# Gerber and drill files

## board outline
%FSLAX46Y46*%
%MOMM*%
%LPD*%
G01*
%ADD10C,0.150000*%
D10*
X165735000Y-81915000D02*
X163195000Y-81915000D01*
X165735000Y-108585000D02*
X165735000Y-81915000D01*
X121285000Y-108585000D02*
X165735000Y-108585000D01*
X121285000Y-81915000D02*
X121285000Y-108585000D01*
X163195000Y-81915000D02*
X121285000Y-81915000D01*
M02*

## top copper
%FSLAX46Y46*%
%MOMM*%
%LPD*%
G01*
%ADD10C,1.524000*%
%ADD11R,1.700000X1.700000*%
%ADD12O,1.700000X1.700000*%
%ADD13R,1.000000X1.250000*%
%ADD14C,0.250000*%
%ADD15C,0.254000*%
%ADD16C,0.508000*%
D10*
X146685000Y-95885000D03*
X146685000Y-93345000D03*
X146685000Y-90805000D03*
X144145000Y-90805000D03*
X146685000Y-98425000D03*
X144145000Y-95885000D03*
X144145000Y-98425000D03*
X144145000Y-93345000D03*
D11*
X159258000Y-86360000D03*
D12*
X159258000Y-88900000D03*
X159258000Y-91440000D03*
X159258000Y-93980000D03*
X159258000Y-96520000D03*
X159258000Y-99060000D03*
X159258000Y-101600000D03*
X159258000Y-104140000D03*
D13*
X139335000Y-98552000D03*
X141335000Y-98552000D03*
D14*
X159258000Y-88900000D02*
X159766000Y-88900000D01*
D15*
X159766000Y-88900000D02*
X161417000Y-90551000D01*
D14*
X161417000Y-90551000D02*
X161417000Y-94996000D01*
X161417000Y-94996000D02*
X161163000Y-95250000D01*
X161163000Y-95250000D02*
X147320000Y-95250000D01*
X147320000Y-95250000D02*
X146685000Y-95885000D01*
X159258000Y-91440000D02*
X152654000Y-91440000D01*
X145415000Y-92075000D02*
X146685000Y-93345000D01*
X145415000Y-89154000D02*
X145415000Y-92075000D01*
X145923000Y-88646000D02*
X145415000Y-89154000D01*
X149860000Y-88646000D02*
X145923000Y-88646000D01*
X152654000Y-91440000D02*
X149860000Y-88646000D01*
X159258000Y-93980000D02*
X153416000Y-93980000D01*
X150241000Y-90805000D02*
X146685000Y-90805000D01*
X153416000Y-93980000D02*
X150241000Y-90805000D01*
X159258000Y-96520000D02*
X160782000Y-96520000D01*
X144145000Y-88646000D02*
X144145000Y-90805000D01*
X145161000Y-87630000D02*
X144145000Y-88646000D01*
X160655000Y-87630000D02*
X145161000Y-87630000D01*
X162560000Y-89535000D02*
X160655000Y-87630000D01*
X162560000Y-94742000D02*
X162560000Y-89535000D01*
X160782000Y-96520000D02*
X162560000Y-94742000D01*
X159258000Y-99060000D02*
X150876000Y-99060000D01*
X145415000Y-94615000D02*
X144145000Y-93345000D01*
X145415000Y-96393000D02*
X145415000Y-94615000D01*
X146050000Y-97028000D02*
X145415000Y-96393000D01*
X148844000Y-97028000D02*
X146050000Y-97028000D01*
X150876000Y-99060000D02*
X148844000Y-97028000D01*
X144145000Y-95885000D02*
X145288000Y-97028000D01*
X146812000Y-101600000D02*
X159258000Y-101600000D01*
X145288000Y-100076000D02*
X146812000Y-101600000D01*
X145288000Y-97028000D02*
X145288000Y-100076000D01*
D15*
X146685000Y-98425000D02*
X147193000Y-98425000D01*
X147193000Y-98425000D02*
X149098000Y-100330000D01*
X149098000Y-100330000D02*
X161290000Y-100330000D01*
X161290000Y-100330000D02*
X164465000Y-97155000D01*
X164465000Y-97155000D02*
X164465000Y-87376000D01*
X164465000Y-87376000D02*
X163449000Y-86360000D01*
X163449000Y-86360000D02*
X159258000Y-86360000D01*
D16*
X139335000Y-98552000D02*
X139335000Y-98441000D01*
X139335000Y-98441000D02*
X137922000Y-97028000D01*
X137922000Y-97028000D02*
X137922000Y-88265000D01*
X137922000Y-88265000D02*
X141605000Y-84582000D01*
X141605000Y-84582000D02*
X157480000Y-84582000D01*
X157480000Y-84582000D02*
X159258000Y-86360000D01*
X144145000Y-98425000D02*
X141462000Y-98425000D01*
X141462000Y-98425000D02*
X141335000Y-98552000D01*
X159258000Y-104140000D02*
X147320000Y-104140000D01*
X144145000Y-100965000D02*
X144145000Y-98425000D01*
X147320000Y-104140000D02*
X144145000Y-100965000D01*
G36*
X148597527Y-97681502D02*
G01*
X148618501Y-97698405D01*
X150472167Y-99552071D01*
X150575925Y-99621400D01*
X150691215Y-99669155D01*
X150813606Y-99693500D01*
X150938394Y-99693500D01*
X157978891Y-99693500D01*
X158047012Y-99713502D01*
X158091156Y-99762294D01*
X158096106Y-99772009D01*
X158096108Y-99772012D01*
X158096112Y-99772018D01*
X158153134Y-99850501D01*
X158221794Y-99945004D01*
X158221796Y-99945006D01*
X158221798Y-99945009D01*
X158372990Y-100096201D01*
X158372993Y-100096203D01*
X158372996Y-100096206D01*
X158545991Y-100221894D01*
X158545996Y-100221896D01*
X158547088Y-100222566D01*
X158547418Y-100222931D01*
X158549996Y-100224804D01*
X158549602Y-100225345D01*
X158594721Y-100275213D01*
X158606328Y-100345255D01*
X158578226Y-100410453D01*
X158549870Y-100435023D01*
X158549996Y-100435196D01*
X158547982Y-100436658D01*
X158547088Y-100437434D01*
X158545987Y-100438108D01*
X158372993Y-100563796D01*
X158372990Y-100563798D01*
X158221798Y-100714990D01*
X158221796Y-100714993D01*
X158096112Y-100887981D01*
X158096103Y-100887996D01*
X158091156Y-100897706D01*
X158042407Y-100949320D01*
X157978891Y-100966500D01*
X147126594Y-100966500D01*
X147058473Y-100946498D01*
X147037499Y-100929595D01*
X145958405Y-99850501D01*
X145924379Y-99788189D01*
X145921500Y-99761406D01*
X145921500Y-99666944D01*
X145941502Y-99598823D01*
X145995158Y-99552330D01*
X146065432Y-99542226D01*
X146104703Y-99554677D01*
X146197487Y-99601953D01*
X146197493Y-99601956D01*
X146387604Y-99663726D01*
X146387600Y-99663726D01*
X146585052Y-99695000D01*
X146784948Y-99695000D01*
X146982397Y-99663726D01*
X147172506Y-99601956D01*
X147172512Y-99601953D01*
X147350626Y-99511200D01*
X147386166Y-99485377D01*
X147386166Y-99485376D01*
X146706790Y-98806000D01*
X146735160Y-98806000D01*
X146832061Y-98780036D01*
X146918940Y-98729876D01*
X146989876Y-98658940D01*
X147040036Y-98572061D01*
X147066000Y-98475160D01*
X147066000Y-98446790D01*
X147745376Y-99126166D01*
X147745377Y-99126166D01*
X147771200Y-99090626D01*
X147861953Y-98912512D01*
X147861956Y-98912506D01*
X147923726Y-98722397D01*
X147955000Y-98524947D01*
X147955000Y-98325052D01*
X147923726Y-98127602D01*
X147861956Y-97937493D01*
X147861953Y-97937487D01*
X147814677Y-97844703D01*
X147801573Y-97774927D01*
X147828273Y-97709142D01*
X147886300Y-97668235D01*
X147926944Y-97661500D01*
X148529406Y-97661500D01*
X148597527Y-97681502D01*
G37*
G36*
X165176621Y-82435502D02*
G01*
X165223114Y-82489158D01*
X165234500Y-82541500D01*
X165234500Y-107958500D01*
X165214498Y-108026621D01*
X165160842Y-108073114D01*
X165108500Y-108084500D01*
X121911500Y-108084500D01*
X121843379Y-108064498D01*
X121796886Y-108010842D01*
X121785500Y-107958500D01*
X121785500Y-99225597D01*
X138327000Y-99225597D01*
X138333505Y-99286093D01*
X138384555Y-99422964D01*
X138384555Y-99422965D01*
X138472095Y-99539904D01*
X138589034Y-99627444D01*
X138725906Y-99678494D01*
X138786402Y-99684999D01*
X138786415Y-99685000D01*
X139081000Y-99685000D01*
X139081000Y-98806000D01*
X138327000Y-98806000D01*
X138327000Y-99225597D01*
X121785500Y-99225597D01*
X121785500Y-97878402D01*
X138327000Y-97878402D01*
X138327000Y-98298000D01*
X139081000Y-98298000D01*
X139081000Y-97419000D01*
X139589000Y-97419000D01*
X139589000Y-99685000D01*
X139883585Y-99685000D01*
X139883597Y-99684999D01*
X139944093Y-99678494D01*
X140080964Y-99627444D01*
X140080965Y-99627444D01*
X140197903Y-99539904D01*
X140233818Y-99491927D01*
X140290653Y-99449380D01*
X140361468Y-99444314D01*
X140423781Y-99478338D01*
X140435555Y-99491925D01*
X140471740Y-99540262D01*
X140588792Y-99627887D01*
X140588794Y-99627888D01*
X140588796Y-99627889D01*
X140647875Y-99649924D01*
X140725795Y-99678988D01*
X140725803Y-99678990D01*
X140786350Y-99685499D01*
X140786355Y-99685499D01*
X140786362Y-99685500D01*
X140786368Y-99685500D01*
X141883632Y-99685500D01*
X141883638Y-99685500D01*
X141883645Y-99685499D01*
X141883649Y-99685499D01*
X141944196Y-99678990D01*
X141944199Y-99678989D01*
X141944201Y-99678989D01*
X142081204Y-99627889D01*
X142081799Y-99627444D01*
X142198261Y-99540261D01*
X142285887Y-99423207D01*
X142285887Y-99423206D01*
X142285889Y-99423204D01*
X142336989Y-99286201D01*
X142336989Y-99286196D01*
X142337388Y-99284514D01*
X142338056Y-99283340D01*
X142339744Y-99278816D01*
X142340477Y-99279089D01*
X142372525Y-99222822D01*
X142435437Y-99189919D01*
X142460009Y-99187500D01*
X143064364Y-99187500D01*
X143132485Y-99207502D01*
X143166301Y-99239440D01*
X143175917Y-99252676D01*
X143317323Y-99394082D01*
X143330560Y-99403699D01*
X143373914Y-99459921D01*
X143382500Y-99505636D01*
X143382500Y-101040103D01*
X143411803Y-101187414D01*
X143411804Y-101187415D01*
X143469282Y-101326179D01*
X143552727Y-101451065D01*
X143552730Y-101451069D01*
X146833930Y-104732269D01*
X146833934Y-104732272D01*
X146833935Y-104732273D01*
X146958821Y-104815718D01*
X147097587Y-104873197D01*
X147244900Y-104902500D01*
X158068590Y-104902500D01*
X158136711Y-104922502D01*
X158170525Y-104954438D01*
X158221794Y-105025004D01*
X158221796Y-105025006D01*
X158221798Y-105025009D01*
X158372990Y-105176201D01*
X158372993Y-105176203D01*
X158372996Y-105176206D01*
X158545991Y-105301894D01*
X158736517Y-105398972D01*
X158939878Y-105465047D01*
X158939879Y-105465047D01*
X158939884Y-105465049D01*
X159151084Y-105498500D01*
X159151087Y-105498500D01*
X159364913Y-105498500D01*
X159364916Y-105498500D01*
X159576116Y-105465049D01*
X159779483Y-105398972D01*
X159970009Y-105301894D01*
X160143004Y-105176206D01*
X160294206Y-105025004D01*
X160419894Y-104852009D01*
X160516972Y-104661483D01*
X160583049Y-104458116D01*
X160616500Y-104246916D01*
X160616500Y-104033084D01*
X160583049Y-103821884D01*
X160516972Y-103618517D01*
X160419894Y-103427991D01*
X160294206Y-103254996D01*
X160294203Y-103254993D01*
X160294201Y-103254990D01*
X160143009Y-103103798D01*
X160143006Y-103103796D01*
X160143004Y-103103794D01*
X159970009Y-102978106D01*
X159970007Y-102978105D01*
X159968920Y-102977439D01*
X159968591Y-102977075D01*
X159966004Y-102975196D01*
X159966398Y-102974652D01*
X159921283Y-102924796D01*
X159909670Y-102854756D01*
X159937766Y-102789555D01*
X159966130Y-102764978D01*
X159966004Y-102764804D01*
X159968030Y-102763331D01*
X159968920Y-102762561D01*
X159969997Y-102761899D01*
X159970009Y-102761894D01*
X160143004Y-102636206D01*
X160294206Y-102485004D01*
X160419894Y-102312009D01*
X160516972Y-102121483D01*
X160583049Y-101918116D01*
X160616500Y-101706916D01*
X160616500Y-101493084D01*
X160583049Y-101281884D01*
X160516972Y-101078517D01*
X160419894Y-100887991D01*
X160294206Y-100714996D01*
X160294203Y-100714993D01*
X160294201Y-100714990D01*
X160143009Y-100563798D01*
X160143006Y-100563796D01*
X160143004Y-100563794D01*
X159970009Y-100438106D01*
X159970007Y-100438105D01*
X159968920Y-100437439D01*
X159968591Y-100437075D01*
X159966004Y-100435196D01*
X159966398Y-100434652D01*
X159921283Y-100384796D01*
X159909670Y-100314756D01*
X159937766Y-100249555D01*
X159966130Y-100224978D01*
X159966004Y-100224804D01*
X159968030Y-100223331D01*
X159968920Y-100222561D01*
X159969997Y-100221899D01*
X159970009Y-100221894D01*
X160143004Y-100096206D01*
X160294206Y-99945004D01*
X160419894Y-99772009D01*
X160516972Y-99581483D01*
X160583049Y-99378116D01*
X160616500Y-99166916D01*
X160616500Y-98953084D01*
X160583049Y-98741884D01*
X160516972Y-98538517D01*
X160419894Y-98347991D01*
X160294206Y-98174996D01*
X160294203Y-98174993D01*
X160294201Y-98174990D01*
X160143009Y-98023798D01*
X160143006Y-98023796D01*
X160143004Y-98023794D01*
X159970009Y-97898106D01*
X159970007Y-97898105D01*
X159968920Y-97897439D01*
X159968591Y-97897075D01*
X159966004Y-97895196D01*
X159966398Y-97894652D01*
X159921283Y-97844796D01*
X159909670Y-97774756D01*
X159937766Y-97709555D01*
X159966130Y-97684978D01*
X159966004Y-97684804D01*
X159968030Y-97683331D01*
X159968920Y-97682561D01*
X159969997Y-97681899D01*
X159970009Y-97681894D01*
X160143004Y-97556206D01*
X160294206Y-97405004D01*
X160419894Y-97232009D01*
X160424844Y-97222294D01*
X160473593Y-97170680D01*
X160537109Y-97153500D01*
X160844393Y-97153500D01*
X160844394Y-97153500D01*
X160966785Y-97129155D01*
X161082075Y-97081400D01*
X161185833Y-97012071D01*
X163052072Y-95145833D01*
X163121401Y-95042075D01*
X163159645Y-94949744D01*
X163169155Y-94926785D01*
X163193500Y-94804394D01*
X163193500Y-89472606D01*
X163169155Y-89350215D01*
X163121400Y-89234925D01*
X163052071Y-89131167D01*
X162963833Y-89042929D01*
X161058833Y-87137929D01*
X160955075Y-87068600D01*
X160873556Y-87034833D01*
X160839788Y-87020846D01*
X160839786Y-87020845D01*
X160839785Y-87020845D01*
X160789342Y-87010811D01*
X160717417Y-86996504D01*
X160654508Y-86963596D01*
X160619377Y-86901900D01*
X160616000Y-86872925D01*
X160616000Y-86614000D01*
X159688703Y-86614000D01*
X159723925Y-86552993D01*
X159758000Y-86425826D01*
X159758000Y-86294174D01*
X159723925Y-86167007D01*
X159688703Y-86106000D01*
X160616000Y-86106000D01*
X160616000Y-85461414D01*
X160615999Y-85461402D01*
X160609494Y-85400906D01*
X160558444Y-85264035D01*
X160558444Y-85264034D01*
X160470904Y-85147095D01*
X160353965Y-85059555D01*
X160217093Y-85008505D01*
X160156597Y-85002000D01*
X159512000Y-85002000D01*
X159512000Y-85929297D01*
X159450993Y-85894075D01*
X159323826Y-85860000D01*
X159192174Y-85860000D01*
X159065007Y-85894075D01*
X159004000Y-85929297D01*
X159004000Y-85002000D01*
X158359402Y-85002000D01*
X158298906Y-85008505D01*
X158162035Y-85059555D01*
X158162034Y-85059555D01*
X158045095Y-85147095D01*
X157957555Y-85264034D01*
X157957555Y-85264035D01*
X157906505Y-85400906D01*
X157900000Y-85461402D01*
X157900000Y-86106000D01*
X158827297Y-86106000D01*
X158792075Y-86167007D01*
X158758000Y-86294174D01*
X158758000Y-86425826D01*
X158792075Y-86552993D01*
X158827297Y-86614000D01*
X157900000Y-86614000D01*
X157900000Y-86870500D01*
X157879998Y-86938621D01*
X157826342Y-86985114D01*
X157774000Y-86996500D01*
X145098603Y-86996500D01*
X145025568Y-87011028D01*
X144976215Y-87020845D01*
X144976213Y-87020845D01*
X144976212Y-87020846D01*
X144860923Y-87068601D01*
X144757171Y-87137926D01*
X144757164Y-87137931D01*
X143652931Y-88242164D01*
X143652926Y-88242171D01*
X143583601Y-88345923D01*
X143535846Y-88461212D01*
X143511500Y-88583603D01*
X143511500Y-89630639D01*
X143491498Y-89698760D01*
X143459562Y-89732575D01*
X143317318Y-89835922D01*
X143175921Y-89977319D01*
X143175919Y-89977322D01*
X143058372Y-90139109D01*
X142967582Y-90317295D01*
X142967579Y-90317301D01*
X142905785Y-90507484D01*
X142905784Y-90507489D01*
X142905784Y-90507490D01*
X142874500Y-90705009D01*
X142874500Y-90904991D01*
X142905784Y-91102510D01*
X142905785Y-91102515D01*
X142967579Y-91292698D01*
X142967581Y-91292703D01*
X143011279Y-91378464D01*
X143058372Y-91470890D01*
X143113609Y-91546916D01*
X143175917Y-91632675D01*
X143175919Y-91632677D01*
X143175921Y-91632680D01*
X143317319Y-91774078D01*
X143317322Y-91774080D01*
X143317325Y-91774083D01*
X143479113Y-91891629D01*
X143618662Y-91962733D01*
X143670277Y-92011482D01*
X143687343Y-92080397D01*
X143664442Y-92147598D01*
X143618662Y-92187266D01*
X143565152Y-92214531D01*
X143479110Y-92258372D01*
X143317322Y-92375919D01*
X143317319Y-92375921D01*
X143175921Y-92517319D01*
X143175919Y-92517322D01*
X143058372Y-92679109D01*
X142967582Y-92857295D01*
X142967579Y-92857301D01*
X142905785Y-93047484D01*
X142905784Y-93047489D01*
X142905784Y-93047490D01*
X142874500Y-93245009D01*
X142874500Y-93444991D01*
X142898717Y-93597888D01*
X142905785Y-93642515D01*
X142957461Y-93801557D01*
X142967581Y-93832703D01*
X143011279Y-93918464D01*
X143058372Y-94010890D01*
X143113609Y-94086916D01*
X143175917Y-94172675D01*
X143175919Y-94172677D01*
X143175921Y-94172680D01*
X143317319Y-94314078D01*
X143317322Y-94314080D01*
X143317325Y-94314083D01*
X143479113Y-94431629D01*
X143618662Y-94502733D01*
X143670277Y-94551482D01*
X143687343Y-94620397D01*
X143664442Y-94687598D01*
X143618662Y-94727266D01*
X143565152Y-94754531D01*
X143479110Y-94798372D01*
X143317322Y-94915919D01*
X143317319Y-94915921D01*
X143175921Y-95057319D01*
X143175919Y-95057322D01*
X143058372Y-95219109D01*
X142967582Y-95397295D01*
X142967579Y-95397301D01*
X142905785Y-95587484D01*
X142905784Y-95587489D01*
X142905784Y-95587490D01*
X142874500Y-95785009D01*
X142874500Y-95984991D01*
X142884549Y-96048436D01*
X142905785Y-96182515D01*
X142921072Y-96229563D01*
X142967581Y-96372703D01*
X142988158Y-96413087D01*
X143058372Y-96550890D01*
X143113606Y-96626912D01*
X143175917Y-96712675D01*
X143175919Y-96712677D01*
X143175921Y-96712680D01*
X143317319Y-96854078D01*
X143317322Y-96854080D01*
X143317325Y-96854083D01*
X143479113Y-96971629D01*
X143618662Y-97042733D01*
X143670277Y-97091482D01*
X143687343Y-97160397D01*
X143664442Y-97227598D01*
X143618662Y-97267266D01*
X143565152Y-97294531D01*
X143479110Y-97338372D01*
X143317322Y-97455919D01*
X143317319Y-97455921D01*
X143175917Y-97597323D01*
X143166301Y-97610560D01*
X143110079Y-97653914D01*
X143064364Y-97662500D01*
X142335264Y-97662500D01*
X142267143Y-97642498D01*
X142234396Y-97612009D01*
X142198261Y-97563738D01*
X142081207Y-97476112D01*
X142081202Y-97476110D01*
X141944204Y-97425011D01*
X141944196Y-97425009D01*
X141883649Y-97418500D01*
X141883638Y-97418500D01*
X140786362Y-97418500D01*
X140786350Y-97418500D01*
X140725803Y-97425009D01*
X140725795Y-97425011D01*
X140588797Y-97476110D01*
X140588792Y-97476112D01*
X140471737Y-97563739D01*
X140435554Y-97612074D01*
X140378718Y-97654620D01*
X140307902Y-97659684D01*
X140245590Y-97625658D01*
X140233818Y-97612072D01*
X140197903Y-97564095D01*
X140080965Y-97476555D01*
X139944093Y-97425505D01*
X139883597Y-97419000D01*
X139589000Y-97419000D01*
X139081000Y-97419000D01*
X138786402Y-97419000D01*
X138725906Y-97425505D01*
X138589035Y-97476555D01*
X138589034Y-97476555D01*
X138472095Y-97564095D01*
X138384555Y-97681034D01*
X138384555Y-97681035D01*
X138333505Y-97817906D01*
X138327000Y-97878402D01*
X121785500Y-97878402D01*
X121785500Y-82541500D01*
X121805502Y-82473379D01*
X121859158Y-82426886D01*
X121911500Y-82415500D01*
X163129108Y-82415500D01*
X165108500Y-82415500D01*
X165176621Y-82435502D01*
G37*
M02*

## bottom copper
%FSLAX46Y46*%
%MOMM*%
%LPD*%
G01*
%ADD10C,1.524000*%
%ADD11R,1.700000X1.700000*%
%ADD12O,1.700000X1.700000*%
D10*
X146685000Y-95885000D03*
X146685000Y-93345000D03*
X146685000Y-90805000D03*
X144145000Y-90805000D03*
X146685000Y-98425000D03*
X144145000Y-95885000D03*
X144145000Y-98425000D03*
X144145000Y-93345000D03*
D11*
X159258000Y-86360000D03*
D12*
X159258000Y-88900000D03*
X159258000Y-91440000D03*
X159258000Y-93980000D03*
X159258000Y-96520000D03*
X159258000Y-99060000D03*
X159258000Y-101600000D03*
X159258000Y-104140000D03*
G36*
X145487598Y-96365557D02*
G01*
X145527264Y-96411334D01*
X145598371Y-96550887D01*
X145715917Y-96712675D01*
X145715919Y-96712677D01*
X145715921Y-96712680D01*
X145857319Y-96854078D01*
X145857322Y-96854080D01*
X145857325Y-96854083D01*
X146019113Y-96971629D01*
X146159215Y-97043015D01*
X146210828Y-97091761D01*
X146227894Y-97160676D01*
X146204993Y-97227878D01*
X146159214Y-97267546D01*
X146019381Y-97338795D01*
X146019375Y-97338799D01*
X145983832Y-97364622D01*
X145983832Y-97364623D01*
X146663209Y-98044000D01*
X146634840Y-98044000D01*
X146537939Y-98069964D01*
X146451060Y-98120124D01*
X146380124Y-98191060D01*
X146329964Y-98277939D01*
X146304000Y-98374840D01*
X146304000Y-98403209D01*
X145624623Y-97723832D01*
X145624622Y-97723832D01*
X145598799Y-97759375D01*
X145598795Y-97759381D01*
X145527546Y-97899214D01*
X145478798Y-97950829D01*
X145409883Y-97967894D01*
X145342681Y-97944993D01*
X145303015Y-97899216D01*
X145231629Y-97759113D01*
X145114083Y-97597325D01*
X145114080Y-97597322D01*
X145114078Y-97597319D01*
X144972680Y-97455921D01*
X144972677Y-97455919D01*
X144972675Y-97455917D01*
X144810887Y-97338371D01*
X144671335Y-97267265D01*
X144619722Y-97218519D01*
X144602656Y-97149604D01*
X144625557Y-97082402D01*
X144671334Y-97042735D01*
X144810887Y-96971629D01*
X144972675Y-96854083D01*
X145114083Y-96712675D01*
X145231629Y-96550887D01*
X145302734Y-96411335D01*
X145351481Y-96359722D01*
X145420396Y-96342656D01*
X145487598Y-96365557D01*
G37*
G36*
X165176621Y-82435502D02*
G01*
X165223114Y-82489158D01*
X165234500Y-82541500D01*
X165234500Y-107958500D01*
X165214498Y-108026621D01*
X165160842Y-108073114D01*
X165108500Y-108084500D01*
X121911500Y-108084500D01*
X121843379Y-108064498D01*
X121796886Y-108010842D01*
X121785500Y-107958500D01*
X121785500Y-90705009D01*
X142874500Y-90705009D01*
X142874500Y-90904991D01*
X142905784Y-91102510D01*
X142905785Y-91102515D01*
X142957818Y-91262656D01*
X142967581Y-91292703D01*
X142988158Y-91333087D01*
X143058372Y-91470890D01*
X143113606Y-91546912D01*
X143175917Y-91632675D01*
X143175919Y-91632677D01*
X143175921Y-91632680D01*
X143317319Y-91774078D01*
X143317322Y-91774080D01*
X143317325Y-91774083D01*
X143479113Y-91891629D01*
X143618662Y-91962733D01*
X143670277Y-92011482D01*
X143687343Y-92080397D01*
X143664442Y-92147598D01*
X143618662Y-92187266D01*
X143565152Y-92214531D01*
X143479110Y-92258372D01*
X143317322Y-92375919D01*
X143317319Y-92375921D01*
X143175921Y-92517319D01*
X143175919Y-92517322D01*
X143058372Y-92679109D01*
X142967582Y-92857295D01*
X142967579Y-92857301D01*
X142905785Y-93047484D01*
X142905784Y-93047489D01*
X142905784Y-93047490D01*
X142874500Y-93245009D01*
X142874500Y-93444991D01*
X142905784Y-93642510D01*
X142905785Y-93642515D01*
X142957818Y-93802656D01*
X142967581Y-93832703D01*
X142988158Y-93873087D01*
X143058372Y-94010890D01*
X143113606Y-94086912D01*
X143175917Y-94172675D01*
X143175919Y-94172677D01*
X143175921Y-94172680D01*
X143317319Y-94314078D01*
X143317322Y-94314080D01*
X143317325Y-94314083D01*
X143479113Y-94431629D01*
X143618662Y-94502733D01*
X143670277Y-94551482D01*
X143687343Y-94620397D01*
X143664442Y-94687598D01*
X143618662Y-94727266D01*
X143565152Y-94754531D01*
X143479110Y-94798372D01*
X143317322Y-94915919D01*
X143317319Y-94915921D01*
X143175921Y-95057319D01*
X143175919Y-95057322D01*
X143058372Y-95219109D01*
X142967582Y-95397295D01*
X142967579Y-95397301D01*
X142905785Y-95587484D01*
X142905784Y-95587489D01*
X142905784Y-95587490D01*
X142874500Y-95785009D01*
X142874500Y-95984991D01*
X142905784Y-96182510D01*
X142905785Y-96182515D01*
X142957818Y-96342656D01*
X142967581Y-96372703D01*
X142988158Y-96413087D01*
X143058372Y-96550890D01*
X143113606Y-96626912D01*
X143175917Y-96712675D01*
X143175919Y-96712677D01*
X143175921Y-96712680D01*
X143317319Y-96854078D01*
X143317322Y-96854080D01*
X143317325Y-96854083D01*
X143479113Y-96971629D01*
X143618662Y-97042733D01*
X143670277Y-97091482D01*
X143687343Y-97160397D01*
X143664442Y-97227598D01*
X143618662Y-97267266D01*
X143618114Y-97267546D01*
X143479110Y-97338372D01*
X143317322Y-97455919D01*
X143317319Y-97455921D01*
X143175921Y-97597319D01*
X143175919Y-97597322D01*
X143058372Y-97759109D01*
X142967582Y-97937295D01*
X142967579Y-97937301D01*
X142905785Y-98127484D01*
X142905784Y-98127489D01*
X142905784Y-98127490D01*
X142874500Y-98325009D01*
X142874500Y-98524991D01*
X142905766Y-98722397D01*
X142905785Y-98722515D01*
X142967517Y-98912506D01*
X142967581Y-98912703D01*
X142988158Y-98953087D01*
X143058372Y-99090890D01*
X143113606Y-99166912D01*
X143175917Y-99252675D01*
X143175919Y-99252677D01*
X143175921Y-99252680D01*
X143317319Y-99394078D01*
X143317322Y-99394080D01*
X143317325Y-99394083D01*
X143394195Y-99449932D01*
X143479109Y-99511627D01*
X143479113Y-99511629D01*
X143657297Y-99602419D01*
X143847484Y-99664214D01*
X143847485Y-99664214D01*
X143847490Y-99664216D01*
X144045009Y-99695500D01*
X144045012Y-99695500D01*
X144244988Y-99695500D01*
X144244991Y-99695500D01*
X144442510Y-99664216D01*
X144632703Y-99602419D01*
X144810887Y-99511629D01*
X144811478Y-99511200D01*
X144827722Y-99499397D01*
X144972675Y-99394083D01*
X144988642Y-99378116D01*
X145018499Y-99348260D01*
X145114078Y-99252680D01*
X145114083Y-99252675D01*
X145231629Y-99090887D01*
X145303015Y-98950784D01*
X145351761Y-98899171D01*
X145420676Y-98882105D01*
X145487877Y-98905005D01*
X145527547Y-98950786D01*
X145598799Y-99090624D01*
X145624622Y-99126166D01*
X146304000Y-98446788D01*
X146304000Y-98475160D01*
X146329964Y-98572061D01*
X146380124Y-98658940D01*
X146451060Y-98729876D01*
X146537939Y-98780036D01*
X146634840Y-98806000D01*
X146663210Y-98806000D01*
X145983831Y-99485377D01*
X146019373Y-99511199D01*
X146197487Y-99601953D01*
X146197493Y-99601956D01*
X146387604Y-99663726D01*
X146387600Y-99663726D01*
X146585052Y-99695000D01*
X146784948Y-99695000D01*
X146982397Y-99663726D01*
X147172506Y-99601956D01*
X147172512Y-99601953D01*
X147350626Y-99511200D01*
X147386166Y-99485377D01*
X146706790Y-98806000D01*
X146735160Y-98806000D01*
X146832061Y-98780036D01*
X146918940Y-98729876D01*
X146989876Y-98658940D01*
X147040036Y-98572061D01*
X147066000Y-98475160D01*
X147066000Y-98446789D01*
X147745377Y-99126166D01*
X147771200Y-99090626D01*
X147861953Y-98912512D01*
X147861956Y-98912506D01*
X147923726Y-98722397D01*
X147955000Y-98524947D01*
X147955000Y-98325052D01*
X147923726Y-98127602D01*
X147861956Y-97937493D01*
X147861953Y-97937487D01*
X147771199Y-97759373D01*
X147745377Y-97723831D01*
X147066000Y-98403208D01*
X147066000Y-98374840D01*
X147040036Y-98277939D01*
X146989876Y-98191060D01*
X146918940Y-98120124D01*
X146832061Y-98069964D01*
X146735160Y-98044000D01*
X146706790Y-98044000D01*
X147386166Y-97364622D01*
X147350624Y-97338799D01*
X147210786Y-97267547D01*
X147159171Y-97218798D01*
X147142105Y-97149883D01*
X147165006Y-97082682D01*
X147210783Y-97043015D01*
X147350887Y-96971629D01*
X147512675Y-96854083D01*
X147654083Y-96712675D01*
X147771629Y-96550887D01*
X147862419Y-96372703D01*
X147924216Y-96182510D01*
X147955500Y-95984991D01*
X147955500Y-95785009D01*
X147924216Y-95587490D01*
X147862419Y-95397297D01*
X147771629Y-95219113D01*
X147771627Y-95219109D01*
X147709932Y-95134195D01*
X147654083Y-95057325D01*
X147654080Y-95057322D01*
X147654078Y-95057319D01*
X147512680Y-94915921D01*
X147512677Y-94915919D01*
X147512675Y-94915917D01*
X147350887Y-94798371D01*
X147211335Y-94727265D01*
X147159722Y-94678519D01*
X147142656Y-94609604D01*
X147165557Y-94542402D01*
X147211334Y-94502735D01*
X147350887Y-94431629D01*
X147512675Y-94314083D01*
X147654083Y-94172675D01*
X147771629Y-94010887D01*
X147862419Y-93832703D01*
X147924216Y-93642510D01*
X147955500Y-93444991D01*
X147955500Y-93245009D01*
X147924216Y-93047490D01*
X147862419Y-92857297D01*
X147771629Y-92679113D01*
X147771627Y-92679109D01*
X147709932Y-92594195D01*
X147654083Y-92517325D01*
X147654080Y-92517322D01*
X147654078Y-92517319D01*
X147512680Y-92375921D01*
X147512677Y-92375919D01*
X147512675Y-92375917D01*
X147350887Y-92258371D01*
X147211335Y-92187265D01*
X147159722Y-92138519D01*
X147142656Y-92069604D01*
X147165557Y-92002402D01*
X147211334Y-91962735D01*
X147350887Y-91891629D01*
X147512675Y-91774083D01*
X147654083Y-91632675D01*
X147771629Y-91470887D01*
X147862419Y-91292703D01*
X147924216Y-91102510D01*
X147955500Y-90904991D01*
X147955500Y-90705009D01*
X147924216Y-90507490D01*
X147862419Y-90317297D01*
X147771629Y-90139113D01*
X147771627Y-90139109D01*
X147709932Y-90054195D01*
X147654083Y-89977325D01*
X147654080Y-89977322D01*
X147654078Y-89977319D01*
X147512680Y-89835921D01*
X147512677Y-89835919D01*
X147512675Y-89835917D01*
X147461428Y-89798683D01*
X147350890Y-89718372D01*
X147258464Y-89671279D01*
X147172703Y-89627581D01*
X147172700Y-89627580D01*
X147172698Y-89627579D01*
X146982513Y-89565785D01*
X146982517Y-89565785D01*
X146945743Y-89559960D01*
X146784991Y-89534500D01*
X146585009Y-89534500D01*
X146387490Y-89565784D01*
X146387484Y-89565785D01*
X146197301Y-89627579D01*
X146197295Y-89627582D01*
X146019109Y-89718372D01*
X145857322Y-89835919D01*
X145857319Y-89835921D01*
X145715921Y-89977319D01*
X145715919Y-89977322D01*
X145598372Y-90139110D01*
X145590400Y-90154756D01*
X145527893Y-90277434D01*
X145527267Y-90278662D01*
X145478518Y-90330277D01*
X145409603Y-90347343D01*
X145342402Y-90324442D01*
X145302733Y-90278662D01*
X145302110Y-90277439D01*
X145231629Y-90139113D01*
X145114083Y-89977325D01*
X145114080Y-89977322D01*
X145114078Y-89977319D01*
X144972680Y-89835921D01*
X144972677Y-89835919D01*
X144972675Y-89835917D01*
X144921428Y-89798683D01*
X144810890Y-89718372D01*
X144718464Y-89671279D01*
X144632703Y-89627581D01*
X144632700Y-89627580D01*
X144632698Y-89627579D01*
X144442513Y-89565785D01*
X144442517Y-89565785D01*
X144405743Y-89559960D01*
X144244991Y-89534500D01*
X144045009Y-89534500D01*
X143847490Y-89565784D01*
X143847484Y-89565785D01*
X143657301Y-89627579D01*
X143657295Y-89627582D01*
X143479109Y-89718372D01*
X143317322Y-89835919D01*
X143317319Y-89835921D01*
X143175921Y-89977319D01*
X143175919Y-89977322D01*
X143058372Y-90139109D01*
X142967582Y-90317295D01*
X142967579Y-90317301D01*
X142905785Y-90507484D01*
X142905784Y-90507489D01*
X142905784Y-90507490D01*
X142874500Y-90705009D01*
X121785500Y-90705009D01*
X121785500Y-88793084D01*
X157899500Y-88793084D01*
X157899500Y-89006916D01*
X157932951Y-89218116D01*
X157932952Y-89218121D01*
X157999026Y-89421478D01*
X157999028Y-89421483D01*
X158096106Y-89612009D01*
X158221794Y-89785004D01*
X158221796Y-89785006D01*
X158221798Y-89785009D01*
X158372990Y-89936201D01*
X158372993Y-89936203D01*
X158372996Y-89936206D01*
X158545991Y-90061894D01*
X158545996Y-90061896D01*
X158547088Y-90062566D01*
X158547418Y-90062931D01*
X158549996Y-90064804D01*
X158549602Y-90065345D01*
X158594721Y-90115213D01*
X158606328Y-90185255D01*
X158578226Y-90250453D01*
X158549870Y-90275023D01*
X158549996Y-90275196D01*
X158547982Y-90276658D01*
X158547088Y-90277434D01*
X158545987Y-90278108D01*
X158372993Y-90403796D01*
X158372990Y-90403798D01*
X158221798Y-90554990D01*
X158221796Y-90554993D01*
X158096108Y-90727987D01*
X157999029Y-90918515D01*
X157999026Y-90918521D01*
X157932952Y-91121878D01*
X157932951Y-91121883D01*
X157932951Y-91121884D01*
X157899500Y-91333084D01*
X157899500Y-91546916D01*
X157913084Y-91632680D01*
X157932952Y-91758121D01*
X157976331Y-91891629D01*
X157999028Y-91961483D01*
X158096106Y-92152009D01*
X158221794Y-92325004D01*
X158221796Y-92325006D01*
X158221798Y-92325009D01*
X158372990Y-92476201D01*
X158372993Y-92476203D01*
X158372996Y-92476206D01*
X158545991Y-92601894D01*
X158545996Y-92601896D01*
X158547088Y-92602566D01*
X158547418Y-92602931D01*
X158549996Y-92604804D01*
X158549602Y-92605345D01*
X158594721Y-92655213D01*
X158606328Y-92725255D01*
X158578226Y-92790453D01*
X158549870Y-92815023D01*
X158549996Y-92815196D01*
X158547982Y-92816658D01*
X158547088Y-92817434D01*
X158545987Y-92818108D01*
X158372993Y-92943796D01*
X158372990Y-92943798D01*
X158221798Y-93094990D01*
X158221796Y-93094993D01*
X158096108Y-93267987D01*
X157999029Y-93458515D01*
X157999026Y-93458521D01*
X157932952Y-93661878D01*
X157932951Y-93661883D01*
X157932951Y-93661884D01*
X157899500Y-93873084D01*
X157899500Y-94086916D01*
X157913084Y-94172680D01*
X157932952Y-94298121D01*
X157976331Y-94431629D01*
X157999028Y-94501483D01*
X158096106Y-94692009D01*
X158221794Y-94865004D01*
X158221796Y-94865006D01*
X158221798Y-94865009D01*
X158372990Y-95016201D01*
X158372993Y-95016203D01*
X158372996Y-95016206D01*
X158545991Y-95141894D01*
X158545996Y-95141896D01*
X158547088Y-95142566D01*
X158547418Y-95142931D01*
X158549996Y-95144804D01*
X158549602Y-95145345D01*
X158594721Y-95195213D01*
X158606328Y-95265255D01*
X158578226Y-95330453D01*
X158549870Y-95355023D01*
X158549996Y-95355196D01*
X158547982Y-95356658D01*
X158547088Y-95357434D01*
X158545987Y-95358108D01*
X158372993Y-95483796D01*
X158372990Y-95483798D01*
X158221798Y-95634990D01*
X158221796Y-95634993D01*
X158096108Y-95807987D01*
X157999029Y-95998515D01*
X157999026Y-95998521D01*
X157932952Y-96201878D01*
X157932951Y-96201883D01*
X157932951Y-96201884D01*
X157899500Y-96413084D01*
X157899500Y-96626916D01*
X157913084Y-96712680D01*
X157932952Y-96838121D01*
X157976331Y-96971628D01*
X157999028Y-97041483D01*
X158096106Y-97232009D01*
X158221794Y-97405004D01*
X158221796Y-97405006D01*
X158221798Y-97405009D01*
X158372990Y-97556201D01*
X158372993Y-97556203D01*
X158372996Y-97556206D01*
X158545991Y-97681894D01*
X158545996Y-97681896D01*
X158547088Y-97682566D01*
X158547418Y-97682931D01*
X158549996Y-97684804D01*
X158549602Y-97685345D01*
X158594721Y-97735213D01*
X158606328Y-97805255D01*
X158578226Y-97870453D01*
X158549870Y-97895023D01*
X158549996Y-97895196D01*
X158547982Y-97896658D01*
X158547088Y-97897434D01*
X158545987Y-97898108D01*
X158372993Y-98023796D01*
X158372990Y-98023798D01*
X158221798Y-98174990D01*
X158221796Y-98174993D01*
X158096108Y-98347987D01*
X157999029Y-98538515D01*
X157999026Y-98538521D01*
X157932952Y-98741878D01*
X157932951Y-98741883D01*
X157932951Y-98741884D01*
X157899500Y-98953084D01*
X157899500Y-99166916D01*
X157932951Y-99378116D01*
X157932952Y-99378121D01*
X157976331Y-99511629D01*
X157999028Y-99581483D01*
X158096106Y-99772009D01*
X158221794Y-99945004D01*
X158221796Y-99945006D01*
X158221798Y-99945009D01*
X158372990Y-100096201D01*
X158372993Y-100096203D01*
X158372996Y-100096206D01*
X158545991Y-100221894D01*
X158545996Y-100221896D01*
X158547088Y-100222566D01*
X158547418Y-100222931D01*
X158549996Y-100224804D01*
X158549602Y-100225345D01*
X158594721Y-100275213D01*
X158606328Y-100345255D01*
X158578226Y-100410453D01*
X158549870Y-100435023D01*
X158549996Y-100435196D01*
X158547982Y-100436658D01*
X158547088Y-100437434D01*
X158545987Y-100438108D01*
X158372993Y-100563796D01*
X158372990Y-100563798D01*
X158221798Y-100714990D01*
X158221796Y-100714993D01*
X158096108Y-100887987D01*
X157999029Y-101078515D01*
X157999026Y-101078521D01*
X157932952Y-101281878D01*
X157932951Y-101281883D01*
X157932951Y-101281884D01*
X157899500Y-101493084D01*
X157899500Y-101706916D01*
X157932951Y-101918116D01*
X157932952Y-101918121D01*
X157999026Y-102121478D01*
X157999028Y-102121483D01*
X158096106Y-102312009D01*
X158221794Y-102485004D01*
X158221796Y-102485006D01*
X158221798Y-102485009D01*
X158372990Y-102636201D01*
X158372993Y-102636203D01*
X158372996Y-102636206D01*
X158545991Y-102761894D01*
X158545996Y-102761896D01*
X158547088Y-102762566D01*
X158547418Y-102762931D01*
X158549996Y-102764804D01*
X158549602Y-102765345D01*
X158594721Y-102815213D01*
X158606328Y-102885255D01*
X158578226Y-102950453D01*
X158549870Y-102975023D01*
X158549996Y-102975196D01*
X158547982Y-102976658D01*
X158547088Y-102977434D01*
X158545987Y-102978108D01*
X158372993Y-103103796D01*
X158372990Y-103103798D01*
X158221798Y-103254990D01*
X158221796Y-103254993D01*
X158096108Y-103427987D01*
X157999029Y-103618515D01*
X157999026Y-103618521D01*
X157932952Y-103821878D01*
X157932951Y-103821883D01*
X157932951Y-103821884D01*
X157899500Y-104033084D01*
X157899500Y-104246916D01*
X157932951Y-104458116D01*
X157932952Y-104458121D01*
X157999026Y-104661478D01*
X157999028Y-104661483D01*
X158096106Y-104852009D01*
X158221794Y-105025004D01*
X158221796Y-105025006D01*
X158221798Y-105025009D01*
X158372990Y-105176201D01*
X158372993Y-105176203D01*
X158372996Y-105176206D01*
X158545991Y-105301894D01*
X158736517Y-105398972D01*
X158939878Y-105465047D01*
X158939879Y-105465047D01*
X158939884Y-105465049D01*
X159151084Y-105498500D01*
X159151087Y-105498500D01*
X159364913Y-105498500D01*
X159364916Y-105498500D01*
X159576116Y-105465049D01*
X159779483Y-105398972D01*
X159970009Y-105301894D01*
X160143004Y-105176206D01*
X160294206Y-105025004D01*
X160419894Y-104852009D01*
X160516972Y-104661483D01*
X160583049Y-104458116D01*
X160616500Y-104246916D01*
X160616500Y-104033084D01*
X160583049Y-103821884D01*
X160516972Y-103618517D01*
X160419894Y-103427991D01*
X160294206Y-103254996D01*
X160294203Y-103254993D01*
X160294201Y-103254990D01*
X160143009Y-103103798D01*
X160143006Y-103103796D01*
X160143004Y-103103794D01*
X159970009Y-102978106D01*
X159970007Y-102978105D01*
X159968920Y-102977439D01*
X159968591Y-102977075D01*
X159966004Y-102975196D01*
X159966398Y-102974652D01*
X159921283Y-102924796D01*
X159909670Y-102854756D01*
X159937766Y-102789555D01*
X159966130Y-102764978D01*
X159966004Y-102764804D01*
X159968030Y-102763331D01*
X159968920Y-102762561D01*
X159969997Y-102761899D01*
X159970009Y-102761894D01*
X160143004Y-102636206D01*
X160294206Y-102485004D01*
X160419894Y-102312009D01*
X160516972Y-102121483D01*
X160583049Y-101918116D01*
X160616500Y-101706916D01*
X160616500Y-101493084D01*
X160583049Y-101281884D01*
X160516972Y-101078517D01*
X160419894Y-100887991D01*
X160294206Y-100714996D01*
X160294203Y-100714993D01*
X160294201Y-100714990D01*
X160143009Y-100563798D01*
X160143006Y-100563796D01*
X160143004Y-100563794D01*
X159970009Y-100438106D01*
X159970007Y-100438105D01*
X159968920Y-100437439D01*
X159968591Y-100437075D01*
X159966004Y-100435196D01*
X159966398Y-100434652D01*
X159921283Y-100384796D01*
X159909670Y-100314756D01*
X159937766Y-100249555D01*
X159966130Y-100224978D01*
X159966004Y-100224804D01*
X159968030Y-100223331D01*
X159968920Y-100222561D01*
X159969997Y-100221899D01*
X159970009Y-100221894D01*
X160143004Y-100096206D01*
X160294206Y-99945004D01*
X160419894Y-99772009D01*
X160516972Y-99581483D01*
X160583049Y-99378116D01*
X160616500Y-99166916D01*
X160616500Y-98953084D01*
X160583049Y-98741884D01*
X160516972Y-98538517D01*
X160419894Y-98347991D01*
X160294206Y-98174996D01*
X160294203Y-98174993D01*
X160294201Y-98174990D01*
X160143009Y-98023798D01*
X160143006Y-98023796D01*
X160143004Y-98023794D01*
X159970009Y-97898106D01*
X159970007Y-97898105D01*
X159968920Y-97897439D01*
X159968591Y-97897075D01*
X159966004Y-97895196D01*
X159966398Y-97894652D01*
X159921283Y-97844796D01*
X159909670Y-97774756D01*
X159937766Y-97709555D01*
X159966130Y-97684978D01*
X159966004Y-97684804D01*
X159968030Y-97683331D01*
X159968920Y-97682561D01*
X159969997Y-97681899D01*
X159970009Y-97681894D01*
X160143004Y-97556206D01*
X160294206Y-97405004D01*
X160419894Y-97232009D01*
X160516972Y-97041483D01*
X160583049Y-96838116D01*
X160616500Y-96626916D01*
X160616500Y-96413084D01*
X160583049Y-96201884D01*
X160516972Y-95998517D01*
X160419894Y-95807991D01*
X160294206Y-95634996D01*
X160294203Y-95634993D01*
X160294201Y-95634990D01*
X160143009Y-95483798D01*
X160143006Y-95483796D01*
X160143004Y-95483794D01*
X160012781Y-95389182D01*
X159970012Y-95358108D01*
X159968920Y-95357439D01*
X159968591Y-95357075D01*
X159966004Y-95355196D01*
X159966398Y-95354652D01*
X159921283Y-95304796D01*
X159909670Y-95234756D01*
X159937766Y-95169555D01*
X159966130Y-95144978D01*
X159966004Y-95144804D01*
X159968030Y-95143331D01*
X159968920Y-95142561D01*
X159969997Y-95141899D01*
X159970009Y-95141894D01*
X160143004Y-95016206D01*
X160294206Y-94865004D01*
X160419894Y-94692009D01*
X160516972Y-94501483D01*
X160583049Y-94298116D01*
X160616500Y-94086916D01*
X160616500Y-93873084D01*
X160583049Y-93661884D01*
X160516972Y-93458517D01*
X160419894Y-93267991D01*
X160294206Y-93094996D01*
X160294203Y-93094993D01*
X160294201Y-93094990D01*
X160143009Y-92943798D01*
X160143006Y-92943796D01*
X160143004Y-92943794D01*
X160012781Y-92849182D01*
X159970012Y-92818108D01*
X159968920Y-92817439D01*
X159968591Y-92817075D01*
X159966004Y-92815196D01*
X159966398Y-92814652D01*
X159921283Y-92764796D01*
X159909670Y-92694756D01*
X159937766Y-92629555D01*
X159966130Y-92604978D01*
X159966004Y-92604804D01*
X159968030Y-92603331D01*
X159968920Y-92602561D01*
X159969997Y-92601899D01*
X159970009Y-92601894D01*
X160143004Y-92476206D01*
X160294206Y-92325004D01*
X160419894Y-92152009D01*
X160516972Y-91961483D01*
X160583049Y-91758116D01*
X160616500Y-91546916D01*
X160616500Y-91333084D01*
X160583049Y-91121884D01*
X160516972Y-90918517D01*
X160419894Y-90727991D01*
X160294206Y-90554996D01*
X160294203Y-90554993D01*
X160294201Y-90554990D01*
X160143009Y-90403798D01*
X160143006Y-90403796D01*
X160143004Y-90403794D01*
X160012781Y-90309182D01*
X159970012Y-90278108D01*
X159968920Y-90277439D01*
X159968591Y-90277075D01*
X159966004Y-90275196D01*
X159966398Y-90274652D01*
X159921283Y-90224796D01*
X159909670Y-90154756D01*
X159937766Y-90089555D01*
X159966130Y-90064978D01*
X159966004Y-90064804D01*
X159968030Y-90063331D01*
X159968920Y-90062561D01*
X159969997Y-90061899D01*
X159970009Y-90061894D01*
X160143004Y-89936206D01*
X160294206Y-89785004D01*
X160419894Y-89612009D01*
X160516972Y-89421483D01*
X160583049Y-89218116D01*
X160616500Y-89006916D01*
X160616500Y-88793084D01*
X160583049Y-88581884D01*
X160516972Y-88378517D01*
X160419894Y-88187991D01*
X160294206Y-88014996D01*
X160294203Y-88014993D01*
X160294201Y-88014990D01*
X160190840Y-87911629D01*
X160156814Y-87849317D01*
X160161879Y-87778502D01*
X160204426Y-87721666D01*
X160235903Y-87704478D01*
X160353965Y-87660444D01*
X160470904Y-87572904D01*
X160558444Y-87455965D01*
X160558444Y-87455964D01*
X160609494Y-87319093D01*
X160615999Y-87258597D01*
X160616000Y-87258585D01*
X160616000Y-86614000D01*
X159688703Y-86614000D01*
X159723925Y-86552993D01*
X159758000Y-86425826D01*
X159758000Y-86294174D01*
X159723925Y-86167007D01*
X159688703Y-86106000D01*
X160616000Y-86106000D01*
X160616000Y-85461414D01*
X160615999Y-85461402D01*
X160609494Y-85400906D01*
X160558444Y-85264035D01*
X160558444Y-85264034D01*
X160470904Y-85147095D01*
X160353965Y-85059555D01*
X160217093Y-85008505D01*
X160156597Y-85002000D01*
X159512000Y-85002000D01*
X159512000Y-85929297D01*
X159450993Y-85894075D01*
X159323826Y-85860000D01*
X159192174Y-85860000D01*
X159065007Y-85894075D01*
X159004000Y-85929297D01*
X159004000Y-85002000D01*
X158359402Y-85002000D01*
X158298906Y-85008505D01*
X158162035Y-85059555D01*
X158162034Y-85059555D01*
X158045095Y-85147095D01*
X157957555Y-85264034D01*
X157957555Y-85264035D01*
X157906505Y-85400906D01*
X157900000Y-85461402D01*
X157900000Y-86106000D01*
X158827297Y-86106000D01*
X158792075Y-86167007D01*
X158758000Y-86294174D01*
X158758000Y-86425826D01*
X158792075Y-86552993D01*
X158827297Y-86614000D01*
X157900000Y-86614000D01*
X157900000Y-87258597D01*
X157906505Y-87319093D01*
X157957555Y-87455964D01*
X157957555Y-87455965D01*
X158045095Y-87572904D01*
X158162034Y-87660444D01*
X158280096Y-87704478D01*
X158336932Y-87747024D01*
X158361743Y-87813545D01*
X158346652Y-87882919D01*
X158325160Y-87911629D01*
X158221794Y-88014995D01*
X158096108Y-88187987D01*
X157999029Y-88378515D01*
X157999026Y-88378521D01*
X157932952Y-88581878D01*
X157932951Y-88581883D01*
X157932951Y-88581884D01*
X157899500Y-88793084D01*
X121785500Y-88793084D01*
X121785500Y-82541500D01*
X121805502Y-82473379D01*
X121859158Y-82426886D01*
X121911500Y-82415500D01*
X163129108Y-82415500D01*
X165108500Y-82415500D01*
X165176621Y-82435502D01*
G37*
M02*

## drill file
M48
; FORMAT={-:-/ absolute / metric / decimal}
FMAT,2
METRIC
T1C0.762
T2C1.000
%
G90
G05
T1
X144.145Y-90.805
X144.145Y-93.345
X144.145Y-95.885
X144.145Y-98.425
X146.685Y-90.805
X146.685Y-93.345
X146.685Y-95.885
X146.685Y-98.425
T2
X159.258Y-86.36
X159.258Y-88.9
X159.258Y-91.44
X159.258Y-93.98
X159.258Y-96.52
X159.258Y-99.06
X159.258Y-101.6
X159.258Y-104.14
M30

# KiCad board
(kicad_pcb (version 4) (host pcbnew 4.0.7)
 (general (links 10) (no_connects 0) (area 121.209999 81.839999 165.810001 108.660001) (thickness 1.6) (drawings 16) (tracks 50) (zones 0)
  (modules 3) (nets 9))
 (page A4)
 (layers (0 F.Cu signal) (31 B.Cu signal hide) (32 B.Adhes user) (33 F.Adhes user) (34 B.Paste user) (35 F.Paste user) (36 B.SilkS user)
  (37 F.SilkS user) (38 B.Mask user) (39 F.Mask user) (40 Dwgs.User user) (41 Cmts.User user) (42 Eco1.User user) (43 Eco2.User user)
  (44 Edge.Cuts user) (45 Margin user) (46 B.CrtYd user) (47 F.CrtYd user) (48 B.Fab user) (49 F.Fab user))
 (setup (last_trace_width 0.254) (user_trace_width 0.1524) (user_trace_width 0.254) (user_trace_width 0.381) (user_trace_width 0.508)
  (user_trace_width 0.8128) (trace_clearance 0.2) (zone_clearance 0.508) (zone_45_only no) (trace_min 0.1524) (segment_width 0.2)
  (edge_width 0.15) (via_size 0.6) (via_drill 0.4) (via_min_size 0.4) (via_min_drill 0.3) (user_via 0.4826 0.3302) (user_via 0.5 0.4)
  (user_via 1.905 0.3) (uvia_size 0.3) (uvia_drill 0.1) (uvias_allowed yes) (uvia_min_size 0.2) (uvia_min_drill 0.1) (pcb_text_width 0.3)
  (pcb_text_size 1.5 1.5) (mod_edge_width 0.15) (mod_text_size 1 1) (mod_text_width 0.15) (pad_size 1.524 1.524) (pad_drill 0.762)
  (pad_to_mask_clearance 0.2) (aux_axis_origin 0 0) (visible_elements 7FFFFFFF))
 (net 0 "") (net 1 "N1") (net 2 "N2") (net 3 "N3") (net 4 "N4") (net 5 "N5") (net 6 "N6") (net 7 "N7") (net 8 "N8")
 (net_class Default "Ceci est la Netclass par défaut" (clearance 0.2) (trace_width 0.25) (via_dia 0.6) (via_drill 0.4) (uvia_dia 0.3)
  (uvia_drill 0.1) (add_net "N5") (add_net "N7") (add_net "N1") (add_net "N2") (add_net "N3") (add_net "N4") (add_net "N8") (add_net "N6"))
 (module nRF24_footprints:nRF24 (layer F.Cu) (at 139.065 95.885)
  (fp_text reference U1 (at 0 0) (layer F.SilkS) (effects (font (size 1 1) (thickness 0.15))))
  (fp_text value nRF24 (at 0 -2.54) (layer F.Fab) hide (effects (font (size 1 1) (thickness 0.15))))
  (pad 1 thru_hole circle (at 7.62 0) (size 1.524 1.524) (drill 0.762) (layers *.Cu *.Mask) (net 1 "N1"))
  (pad 2 thru_hole circle (at 7.62 -2.54) (size 1.524 1.524) (drill 0.762) (layers *.Cu *.Mask) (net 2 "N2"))
  (pad 3 thru_hole circle (at 7.62 -5.08) (size 1.524 1.524) (drill 0.762) (layers *.Cu *.Mask) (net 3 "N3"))
  (pad 4 thru_hole circle (at 5.08 -5.08) (size 1.524 1.524) (drill 0.762) (layers *.Cu *.Mask) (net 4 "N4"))
  (pad 0 thru_hole circle (at 7.62 2.54) (size 1.524 1.524) (drill 0.762) (layers *.Cu *.Mask) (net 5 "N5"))
  (pad 6 thru_hole circle (at 5.08 0) (size 1.524 1.524) (drill 0.762) (layers *.Cu *.Mask) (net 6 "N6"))
  (pad 7 thru_hole circle (at 5.08 2.54) (size 1.524 1.524) (drill 0.762) (layers *.Cu *.Mask) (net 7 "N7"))
  (pad 5 thru_hole circle (at 5.08 -2.54) (size 1.524 1.524) (drill 0.762) (layers *.Cu *.Mask) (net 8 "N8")))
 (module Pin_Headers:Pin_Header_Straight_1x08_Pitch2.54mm (layer F.Cu) (at 159.258 86.36)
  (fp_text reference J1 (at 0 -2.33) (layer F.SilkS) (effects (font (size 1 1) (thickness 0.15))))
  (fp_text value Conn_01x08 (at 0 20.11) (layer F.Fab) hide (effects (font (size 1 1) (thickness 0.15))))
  (pad 1 thru_hole rect (at 0 0) (size 1.7 1.7) (drill 1) (layers *.Cu *.Mask) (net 5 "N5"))
  (pad 2 thru_hole oval (at 0 2.54) (size 1.7 1.7) (drill 1) (layers *.Cu *.Mask) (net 1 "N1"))
  (pad 3 thru_hole oval (at 0 5.08) (size 1.7 1.7) (drill 1) (layers *.Cu *.Mask) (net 2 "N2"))
  (pad 4 thru_hole oval (at 0 7.62) (size 1.7 1.7) (drill 1) (layers *.Cu *.Mask) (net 3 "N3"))
  (pad 5 thru_hole oval (at 0 10.16) (size 1.7 1.7) (drill 1) (layers *.Cu *.Mask) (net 4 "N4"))
  (pad 6 thru_hole oval (at 0 12.7) (size 1.7 1.7) (drill 1) (layers *.Cu *.Mask) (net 8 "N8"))
  (pad 7 thru_hole oval (at 0 15.24) (size 1.7 1.7) (drill 1) (layers *.Cu *.Mask) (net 6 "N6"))
  (pad 8 thru_hole oval (at 0 17.78) (size 1.7 1.7) (drill 1) (layers *.Cu *.Mask) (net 7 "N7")))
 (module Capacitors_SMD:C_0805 (layer F.Cu) (at 140.335 98.552)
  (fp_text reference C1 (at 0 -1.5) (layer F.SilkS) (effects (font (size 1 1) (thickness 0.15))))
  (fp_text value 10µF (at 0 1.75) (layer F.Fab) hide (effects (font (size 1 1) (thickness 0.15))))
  (pad 1 smd rect (at -1 0) (size 1 1.25) (layers F.Cu F.Paste F.Mask) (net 5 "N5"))
  (pad 2 smd rect (at 1 0) (size 1 1.25) (layers F.Cu F.Paste F.Mask) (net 7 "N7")))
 (gr_line (start 165.735 81.915) (end 163.195 81.915) (angle 90) (layer Edge.Cuts) (width 0.15))
 (gr_line (start 165.735 108.585) (end 165.735 81.915) (angle 90) (layer Edge.Cuts) (width 0.15))
 (gr_line (start 121.285 108.585) (end 165.735 108.585) (angle 90) (layer Edge.Cuts) (width 0.15))
 (gr_line (start 121.285 81.915) (end 121.285 108.585) (angle 90) (layer Edge.Cuts) (width 0.15))
 (gr_line (start 163.195 81.915) (end 121.285 81.915) (angle 90) (layer Edge.Cuts) (width 0.15))
 (segment (start 159.258 88.9) (end 159.766 88.9) (width 0.25) (layer F.Cu) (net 1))
 (segment (start 159.766 88.9) (end 161.417 90.551) (width 0.254) (layer F.Cu) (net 1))
 (segment (start 161.417 90.551) (end 161.417 94.996) (width 0.25) (layer F.Cu) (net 1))
 (segment (start 161.417 94.996) (end 161.163 95.25) (width 0.25) (layer F.Cu) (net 1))
 (segment (start 161.163 95.25) (end 147.32 95.25) (width 0.25) (layer F.Cu) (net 1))
 (segment (start 147.32 95.25) (end 146.685 95.885) (width 0.25) (layer F.Cu) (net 1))
 (segment (start 159.258 91.44) (end 152.654 91.44) (width 0.25) (layer F.Cu) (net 2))
 (segment (start 145.415 92.075) (end 146.685 93.345) (width 0.25) (layer F.Cu) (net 2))
 (segment (start 145.415 89.154) (end 145.415 92.075) (width 0.25) (layer F.Cu) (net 2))
 (segment (start 145.923 88.646) (end 145.415 89.154) (width 0.25) (layer F.Cu) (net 2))
 (segment (start 149.86 88.646) (end 145.923 88.646) (width 0.25) (layer F.Cu) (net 2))
 (segment (start 152.654 91.44) (end 149.86 88.646) (width 0.25) (layer F.Cu) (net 2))
 (segment (start 159.258 93.98) (end 153.416 93.98) (width 0.25) (layer F.Cu) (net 3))
 (segment (start 150.241 90.805) (end 146.685 90.805) (width 0.25) (layer F.Cu) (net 3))
 (segment (start 153.416 93.98) (end 150.241 90.805) (width 0.25) (layer F.Cu) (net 3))
 (segment (start 159.258 96.52) (end 160.782 96.52) (width 0.25) (layer F.Cu) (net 4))
 (segment (start 144.145 88.646) (end 144.145 90.805) (width 0.25) (layer F.Cu) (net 4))
 (segment (start 145.161 87.63) (end 144.145 88.646) (width 0.25) (layer F.Cu) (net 4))
 (segment (start 160.655 87.63) (end 145.161 87.63) (width 0.25) (layer F.Cu) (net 4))
 (segment (start 162.56 89.535) (end 160.655 87.63) (width 0.25) (layer F.Cu) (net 4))
 (segment (start 162.56 94.742) (end 162.56 89.535) (width 0.25) (layer F.Cu) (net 4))
 (segment (start 160.782 96.52) (end 162.56 94.742) (width 0.25) (layer F.Cu) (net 4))
 (segment (start 159.258 99.06) (end 150.876 99.06) (width 0.25) (layer F.Cu) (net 8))
 (segment (start 145.415 94.615) (end 144.145 93.345) (width 0.25) (layer F.Cu) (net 8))
 (segment (start 145.415 96.393) (end 145.415 94.615) (width 0.25) (layer F.Cu) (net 8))
 (segment (start 146.05 97.028) (end 145.415 96.393) (width 0.25) (layer F.Cu) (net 8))
 (segment (start 148.844 97.028) (end 146.05 97.028) (width 0.25) (layer F.Cu) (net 8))
 (segment (start 150.876 99.06) (end 148.844 97.028) (width 0.25) (layer F.Cu) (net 8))
 (segment (start 144.145 95.885) (end 145.288 97.028) (width 0.25) (layer F.Cu) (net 6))
 (segment (start 146.812 101.6) (end 159.258 101.6) (width 0.25) (layer F.Cu) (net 6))
 (segment (start 145.288 100.076) (end 146.812 101.6) (width 0.25) (layer F.Cu) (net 6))
 (segment (start 145.288 97.028) (end 145.288 100.076) (width 0.25) (layer F.Cu) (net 6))
 (segment (start 146.685 98.425) (end 147.193 98.425) (width 0.254) (layer F.Cu) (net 5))
 (segment (start 147.193 98.425) (end 149.098 100.33) (width 0.254) (layer F.Cu) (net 5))
 (segment (start 149.098 100.33) (end 161.29 100.33) (width 0.254) (layer F.Cu) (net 5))
 (segment (start 161.29 100.33) (end 164.465 97.155) (width 0.254) (layer F.Cu) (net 5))
 (segment (start 164.465 97.155) (end 164.465 87.376) (width 0.254) (layer F.Cu) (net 5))
 (segment (start 164.465 87.376) (end 163.449 86.36) (width 0.254) (layer F.Cu) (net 5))
 (segment (start 163.449 86.36) (end 159.258 86.36) (width 0.254) (layer F.Cu) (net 5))
 (segment (start 139.335 98.552) (end 139.335 98.441) (width 0.508) (layer F.Cu) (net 5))
 (segment (start 139.335 98.441) (end 137.922 97.028) (width 0.508) (layer F.Cu) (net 5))
 (segment (start 137.922 97.028) (end 137.922 88.265) (width 0.508) (layer F.Cu) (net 5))
 (segment (start 137.922 88.265) (end 141.605 84.582) (width 0.508) (layer F.Cu) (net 5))
 (segment (start 141.605 84.582) (end 157.48 84.582) (width 0.508) (layer F.Cu) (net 5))
 (segment (start 157.48 84.582) (end 159.258 86.36) (width 0.508) (layer F.Cu) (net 5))
 (segment (start 144.145 98.425) (end 141.462 98.425) (width 0.508) (layer F.Cu) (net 7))
 (segment (start 141.462 98.425) (end 141.335 98.552) (width 0.508) (layer F.Cu) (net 7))
 (segment (start 159.258 104.14) (end 147.32 104.14) (width 0.508) (layer F.Cu) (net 7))
 (segment (start 144.145 100.965) (end 144.145 98.425) (width 0.508) (layer F.Cu) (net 7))
 (segment (start 147.32 104.14) (end 144.145 100.965) (width 0.508) (layer F.Cu) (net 7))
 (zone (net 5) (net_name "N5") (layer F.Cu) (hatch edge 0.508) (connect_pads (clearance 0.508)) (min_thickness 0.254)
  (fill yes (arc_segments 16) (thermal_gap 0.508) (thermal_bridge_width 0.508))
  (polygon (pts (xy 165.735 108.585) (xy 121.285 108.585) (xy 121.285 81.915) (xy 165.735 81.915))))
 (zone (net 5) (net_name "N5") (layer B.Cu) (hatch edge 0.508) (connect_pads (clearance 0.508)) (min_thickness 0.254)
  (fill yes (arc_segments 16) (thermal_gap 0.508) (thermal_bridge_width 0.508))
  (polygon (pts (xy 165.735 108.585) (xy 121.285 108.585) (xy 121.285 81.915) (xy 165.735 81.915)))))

